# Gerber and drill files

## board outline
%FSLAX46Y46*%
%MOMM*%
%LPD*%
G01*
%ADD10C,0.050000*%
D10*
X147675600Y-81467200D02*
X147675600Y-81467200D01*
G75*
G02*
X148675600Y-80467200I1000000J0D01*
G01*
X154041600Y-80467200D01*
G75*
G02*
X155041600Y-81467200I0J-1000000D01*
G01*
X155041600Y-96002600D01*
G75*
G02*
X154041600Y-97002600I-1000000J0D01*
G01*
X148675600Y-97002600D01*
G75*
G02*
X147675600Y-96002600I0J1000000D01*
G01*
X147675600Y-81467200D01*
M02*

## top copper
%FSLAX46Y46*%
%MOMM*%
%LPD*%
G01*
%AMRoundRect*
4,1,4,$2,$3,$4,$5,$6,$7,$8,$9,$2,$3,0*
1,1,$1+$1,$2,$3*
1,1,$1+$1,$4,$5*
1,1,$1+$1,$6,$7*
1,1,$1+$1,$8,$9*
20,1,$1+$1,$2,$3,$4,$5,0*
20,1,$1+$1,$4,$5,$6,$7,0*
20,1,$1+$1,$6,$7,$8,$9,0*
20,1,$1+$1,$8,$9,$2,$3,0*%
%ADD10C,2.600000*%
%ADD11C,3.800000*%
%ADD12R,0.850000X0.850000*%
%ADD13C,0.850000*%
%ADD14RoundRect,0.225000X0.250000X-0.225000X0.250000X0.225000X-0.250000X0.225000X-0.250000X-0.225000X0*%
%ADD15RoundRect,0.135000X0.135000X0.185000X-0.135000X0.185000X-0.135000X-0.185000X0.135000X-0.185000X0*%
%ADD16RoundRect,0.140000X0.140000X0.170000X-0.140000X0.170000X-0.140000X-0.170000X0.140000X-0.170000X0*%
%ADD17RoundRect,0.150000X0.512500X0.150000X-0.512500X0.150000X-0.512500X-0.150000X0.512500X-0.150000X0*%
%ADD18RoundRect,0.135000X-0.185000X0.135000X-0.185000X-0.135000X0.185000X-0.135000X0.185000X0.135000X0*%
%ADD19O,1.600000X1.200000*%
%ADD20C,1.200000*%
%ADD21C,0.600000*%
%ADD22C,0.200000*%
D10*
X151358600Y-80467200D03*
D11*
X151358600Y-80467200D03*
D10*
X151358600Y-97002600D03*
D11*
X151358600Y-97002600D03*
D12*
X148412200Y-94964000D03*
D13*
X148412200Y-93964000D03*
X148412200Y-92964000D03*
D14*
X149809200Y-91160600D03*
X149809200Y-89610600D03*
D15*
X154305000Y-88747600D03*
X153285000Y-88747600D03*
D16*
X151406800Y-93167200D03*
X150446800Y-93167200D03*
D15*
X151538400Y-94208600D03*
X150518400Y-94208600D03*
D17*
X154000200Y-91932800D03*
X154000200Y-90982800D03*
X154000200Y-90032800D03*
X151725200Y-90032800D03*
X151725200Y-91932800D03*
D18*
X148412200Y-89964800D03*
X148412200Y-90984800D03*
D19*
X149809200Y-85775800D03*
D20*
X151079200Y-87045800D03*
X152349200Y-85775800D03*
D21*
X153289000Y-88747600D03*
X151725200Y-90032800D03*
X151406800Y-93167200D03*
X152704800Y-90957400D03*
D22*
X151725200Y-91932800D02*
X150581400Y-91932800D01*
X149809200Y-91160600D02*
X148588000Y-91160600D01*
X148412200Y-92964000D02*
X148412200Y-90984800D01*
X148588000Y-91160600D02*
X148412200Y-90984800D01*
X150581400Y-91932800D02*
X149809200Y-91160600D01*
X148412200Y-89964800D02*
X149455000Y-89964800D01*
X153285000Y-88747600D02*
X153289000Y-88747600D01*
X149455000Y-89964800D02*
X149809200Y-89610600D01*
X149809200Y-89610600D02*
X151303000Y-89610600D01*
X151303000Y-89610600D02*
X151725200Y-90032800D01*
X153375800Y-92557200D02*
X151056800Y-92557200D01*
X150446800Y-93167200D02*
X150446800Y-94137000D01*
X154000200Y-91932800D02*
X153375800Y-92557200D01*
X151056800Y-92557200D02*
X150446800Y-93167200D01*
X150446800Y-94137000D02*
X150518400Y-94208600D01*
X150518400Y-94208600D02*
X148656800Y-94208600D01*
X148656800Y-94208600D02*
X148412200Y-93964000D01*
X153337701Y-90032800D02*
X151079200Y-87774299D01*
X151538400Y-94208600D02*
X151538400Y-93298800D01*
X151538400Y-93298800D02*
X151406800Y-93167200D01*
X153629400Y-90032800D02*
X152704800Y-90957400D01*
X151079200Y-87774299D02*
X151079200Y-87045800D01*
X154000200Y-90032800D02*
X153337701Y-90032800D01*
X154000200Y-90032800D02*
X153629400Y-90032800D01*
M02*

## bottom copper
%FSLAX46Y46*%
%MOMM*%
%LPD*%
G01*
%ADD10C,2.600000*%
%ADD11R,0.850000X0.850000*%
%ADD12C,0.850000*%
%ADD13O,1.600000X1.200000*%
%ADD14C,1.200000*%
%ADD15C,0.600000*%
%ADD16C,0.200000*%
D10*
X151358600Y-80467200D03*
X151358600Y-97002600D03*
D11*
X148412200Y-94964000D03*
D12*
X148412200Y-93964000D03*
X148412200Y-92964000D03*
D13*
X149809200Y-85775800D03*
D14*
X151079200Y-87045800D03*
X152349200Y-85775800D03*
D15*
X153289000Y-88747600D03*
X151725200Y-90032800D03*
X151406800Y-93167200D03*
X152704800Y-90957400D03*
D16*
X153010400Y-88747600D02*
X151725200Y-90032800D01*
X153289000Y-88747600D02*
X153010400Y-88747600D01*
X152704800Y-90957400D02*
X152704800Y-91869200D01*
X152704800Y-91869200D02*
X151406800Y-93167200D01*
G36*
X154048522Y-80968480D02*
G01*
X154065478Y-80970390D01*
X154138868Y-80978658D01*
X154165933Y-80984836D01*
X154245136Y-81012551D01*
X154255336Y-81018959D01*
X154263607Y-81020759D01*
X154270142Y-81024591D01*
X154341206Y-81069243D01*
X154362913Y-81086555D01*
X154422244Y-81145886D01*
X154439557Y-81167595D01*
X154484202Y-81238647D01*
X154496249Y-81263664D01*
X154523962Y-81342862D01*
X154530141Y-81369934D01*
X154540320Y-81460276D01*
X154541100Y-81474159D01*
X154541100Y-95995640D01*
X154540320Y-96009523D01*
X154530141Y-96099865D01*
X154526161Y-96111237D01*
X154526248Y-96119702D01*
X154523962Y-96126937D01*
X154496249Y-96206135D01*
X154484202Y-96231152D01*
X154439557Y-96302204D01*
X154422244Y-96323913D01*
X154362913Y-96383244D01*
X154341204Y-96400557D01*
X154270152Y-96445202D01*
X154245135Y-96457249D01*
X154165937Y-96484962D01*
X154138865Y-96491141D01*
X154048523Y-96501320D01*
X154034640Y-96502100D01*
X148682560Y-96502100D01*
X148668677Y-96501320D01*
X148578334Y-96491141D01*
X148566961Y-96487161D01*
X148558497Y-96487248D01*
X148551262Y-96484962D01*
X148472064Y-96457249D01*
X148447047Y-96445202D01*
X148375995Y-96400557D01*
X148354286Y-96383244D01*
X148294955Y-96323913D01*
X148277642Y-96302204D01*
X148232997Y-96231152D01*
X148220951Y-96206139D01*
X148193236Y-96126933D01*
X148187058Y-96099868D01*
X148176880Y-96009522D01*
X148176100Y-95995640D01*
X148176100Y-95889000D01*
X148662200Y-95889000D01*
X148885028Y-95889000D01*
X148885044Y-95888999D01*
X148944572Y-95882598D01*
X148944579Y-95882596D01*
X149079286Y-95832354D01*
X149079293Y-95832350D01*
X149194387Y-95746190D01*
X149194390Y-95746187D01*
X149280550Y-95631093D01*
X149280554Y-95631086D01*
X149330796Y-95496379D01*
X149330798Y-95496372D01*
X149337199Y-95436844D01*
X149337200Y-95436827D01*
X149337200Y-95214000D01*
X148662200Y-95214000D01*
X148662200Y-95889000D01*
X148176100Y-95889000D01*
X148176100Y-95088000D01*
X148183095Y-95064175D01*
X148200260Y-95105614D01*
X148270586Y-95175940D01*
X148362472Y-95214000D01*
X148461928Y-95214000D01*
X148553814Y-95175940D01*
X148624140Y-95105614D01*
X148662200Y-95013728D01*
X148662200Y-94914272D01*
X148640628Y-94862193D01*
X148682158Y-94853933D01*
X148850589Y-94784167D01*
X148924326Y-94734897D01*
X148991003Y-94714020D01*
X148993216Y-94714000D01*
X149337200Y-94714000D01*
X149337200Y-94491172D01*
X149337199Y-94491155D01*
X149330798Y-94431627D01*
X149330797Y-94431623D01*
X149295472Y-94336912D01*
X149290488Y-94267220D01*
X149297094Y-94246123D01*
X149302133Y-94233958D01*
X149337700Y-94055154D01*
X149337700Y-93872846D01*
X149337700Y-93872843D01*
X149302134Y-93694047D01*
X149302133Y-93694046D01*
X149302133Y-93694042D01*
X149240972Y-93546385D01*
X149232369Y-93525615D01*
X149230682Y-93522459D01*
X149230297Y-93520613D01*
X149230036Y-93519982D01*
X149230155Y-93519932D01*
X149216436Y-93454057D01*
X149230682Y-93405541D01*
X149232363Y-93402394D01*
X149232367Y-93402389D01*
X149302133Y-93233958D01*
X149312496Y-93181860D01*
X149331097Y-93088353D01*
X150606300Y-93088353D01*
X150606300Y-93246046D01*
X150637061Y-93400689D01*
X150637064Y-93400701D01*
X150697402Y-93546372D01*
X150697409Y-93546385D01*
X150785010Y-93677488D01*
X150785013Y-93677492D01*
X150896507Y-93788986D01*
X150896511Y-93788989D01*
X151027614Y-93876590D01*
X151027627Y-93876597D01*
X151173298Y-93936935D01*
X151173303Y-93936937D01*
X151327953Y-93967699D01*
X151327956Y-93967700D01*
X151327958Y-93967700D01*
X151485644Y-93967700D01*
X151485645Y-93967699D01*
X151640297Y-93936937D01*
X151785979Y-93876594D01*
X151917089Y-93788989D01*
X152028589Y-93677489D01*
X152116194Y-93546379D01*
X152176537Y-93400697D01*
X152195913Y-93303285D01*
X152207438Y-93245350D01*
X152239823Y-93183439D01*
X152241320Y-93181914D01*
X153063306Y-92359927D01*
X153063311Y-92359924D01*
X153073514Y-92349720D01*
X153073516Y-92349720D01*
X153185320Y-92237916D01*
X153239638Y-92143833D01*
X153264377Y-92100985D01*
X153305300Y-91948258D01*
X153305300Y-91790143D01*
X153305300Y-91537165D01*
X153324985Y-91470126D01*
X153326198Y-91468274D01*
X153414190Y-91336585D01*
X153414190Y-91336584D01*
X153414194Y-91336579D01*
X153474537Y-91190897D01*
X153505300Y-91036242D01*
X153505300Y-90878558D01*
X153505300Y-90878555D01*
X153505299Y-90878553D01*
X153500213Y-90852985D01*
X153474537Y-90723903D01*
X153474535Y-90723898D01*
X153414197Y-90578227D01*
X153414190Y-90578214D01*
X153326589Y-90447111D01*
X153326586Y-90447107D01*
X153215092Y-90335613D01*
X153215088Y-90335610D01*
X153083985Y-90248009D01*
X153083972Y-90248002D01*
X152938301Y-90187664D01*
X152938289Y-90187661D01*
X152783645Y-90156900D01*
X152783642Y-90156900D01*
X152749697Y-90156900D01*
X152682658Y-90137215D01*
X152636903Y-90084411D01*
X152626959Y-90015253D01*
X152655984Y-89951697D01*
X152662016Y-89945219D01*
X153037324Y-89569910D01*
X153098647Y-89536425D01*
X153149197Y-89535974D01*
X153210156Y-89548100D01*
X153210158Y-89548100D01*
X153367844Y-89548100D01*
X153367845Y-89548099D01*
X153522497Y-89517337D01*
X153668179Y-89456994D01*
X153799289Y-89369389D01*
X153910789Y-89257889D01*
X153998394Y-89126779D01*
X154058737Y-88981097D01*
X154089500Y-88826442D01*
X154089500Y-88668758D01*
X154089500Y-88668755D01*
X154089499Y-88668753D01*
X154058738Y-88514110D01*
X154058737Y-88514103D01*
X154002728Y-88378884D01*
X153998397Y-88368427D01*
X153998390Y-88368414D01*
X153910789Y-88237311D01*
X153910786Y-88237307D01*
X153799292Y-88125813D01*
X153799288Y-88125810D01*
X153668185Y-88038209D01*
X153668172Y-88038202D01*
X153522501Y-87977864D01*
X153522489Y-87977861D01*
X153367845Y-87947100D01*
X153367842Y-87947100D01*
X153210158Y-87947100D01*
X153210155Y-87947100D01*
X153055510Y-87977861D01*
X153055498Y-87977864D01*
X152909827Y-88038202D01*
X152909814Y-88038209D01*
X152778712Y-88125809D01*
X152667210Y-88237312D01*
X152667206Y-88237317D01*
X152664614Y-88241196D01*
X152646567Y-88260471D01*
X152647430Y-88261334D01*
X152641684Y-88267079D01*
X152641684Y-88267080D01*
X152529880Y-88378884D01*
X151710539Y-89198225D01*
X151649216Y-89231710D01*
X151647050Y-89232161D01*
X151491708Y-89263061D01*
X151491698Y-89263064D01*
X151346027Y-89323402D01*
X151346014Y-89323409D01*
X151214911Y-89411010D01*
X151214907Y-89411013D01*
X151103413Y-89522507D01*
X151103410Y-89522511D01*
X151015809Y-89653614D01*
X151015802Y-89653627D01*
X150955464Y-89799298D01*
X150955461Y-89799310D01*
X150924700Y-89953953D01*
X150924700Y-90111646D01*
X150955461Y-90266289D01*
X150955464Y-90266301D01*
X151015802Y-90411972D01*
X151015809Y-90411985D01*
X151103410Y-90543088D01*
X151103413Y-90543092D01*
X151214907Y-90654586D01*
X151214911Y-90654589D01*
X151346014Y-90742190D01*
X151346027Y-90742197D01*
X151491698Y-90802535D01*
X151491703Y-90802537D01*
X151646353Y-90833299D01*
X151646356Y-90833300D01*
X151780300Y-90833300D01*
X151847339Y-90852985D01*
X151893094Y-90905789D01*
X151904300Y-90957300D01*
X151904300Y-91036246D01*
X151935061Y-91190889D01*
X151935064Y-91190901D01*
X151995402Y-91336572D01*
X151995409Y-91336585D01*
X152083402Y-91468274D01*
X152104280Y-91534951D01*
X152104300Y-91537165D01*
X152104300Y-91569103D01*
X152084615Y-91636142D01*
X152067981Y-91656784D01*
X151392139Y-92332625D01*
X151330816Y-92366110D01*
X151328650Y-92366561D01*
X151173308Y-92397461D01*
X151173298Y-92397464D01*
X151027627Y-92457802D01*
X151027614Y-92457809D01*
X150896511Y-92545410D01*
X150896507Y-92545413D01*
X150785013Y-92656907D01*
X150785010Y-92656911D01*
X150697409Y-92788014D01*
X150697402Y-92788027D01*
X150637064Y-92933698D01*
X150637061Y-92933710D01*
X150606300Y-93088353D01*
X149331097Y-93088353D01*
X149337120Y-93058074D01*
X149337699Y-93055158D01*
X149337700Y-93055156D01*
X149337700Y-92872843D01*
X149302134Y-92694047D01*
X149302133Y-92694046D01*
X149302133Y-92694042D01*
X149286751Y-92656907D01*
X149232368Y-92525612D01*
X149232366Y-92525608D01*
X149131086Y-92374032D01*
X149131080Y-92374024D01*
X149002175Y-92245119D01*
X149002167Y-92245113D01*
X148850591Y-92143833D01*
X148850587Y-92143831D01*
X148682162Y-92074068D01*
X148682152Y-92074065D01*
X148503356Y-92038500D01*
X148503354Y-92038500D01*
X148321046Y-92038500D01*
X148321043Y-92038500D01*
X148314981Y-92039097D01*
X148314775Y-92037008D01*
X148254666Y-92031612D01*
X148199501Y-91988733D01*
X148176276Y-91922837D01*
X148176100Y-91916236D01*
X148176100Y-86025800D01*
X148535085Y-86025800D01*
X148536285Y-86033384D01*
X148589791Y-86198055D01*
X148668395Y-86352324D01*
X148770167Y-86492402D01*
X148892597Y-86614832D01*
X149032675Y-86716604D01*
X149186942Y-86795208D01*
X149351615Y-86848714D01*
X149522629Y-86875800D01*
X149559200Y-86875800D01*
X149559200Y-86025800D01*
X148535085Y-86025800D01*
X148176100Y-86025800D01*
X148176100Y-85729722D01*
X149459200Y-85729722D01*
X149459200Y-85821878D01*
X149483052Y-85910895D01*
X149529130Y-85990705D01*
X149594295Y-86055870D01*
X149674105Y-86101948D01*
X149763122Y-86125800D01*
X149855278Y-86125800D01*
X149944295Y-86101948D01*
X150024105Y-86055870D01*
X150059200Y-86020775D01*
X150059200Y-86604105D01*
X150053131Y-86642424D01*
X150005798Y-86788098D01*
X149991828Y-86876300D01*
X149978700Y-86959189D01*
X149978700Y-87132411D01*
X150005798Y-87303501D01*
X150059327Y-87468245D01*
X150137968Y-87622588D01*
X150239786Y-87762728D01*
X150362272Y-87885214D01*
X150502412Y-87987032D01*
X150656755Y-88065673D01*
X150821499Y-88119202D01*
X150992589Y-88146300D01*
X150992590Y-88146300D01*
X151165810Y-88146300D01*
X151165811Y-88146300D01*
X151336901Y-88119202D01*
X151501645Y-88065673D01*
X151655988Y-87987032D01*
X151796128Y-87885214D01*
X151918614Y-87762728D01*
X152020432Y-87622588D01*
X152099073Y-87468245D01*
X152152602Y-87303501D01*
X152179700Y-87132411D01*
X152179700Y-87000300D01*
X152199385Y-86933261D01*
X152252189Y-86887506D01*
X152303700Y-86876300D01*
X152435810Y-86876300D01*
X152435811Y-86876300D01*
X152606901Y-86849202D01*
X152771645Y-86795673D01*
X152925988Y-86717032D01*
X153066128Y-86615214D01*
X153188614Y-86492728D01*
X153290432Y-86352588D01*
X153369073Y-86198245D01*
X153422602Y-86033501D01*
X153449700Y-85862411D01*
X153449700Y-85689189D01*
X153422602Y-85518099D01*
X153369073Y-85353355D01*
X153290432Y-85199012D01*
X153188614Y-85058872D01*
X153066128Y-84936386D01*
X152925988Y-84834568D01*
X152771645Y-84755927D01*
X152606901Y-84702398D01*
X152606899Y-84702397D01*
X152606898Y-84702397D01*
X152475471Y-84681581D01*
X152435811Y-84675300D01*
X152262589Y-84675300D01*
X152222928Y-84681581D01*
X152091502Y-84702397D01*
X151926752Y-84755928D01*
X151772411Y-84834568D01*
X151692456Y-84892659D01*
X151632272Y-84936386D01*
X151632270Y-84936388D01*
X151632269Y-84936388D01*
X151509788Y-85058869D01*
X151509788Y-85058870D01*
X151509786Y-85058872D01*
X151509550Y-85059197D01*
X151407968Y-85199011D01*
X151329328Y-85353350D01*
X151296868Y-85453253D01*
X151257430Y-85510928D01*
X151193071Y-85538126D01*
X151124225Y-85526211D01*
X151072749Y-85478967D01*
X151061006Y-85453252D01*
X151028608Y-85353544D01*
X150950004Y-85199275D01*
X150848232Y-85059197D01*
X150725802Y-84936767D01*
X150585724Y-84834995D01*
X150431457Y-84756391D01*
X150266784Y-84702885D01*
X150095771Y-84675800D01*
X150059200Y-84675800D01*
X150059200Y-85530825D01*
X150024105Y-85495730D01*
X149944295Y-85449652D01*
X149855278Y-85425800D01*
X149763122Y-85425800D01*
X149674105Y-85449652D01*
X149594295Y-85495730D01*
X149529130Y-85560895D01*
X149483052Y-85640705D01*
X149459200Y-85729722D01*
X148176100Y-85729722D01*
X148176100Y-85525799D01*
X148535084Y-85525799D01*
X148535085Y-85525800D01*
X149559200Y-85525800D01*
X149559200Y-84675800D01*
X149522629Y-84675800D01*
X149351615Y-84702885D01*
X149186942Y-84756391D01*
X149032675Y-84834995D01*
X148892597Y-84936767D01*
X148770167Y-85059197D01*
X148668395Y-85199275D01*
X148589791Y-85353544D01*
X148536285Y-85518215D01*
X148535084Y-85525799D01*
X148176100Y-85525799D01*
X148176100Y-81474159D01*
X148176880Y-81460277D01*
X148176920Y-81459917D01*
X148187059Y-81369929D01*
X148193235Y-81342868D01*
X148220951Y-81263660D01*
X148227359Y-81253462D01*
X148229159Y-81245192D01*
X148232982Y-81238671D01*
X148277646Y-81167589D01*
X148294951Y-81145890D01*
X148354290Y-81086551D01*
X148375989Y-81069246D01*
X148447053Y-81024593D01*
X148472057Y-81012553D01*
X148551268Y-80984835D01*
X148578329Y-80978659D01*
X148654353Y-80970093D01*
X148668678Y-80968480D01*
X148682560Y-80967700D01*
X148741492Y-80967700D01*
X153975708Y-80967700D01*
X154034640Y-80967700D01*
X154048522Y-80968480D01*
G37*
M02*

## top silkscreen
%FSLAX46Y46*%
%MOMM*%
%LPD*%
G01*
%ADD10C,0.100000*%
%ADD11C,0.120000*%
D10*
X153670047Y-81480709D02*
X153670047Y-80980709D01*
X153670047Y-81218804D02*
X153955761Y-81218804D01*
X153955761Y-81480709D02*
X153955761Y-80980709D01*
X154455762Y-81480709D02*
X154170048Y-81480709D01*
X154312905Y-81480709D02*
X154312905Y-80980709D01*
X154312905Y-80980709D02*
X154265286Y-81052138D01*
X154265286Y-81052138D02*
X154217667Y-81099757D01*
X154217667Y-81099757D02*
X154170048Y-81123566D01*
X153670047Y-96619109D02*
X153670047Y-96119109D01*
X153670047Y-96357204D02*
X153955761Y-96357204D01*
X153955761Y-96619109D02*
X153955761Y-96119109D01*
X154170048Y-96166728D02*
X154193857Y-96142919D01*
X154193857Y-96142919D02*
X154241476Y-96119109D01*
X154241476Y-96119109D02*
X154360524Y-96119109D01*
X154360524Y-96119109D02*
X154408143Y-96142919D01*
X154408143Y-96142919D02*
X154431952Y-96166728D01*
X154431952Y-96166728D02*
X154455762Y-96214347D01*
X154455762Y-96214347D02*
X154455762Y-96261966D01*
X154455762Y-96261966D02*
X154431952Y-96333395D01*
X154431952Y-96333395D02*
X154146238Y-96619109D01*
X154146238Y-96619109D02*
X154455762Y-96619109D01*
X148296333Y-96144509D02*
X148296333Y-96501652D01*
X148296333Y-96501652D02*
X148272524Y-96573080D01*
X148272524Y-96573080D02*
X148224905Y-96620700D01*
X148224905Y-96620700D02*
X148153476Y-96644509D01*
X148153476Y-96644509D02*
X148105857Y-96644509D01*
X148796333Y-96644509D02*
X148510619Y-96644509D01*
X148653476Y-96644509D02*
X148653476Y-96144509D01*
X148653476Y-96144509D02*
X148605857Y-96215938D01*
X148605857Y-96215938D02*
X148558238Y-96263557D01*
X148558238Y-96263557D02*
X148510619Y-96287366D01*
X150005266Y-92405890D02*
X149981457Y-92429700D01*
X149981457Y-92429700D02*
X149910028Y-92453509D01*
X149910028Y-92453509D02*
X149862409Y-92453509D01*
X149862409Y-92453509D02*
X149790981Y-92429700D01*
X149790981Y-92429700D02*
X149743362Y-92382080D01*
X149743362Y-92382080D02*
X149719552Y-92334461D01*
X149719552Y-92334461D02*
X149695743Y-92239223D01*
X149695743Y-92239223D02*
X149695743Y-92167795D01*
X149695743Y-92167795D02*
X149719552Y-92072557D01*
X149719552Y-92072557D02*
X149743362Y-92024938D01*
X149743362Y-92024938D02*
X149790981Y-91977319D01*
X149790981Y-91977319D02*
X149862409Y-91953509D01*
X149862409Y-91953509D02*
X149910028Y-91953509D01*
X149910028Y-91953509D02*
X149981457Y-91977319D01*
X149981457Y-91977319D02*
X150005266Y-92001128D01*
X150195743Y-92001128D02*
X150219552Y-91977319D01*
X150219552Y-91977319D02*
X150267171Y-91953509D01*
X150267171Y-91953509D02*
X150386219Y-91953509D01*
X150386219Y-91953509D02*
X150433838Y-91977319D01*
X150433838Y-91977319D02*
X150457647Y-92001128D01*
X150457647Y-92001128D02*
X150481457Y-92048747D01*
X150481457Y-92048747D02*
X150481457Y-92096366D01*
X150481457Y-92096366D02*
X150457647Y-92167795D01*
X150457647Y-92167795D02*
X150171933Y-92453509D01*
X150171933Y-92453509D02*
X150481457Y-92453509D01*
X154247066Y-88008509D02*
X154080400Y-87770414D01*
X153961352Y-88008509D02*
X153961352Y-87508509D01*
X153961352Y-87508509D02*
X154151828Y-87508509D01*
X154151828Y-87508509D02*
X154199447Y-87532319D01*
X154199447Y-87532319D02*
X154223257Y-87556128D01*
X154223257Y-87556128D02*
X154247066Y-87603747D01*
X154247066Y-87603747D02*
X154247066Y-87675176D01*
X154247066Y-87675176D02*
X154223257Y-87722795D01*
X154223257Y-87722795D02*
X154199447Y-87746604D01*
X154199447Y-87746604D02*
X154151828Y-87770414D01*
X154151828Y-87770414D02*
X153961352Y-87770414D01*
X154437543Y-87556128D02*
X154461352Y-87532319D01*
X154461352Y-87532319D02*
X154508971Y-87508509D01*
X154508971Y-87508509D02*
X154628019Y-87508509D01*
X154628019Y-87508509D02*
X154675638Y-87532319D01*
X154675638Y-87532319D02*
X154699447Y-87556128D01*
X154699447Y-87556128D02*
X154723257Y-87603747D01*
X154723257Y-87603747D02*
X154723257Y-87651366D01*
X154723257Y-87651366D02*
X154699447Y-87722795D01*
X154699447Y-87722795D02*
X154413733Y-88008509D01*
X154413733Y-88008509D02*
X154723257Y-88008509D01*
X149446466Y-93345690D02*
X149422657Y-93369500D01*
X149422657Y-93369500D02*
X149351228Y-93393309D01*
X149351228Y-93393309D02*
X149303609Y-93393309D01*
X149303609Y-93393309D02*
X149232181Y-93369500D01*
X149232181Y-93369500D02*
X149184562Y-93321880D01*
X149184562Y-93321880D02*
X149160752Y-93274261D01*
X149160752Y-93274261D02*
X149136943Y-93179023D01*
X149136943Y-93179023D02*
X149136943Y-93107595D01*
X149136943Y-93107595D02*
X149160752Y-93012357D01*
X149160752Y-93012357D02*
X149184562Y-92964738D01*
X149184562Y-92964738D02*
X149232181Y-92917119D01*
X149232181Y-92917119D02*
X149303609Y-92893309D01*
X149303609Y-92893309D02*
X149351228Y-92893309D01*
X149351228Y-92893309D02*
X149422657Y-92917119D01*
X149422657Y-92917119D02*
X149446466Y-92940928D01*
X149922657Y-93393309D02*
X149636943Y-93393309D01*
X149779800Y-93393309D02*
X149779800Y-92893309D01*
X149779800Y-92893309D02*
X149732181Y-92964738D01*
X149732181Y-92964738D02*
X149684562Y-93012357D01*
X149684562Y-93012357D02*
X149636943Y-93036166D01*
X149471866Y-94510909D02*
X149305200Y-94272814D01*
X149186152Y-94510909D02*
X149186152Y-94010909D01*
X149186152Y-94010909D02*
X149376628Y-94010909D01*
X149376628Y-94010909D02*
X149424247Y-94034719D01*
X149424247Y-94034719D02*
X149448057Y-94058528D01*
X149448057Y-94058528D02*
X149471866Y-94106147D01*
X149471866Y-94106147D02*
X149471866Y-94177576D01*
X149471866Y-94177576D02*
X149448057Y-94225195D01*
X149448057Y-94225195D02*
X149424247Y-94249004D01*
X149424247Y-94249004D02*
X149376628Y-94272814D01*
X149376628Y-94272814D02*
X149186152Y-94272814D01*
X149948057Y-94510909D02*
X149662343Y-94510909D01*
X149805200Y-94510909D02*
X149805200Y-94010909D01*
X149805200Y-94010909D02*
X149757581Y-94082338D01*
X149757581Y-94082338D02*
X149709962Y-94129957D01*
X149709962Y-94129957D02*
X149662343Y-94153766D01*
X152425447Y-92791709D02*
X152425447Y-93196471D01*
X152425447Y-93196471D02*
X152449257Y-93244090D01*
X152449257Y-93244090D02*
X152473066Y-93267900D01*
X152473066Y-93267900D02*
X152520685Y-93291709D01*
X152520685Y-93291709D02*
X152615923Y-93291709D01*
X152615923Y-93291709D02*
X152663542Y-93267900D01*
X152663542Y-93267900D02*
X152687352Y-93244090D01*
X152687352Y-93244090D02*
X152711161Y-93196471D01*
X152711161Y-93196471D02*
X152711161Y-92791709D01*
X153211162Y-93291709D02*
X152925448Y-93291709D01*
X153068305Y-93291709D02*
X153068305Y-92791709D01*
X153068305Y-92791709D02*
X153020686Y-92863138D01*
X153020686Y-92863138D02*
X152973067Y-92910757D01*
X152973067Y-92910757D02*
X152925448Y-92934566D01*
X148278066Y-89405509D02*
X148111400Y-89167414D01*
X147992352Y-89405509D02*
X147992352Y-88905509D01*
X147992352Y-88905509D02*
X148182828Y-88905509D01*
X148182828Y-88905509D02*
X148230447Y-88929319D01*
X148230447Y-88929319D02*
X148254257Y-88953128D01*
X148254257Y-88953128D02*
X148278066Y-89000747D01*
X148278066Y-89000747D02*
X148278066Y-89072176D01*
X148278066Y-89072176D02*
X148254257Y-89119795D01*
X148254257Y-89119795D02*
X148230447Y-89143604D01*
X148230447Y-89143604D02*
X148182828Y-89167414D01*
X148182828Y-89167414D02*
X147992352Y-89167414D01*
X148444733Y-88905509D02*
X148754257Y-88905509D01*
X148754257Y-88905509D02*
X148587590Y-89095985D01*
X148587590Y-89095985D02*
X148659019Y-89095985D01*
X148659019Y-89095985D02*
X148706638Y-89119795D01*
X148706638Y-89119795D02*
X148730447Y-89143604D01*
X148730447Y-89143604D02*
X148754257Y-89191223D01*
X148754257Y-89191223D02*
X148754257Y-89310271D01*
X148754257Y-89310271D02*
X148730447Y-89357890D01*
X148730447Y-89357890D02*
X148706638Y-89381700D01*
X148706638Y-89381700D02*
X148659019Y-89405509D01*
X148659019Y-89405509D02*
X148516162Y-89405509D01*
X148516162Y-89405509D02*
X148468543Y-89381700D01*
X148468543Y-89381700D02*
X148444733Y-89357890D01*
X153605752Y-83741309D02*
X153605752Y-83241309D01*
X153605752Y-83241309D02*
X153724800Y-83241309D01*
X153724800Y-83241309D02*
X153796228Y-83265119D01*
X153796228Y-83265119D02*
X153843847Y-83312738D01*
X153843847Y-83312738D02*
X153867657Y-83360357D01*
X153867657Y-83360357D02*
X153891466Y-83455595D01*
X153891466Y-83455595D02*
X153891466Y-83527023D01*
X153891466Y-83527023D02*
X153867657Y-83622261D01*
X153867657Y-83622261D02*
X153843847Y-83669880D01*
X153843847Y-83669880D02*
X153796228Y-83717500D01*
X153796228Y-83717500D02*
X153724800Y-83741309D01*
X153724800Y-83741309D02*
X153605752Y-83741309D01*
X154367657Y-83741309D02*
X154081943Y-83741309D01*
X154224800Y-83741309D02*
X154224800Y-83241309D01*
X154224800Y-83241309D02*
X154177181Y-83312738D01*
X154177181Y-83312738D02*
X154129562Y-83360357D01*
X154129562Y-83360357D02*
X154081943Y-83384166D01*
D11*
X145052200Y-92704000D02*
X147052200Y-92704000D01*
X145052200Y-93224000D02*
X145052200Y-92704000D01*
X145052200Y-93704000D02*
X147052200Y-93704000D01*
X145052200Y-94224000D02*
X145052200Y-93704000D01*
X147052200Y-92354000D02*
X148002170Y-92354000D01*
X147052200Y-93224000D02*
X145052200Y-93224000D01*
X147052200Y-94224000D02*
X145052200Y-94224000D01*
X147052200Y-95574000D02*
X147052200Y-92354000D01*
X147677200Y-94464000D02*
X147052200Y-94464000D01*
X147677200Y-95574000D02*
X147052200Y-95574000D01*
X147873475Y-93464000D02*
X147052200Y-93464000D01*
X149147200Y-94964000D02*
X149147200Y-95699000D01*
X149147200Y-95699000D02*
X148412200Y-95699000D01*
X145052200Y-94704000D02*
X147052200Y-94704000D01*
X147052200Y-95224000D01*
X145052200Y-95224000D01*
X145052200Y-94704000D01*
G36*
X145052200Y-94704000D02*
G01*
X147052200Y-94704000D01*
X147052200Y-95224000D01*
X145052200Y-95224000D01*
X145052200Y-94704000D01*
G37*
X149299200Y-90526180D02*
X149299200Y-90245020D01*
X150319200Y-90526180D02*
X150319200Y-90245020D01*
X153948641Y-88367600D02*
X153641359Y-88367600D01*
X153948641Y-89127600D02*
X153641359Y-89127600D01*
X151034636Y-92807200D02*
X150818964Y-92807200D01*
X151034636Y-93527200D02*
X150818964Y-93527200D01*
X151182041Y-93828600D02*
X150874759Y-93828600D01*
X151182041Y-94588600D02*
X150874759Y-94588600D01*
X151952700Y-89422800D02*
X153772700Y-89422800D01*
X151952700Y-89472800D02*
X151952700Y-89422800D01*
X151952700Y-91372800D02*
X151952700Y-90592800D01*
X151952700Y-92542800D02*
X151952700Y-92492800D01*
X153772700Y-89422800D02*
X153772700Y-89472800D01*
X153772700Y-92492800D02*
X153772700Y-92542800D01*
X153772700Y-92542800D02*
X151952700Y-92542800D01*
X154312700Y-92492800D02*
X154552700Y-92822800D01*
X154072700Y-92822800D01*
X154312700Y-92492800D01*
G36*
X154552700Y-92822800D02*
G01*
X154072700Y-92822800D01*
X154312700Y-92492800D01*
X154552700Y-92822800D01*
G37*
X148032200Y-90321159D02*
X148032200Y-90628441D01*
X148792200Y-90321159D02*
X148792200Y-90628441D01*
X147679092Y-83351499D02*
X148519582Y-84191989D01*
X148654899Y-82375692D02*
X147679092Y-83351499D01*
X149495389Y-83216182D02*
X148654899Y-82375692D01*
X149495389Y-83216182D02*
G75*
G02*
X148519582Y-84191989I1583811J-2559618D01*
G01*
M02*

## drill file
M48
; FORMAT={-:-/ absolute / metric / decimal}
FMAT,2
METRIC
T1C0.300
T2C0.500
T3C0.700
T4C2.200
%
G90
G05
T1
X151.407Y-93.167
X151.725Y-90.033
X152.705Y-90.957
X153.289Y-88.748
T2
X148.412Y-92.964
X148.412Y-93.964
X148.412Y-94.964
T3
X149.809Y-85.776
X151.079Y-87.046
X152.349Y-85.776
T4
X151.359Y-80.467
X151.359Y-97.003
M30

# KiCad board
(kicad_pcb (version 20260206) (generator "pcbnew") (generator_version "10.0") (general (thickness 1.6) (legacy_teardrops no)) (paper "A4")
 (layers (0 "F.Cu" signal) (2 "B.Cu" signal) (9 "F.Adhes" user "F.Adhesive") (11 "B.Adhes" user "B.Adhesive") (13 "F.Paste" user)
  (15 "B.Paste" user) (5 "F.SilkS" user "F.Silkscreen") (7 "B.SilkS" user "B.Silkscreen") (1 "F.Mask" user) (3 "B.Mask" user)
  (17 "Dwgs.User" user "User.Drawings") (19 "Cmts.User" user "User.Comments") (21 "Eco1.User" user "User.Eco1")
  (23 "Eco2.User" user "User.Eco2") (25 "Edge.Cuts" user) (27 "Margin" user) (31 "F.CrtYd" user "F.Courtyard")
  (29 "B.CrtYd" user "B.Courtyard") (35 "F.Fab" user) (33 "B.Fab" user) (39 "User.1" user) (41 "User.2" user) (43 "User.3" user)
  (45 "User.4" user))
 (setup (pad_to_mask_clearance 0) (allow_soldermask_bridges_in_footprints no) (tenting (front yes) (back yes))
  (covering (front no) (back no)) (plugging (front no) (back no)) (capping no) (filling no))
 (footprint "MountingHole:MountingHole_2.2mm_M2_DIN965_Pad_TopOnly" (layer "F.Cu") (at 151.3586 80.4672)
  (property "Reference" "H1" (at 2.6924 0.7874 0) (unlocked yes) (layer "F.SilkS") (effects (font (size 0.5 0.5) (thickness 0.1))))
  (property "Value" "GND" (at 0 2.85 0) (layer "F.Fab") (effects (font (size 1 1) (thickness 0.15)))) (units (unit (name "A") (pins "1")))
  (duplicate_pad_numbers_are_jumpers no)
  (pad "1" thru_hole circle (at 0 0) (size 2.6 2.6) (drill 2.2) (layers "*.Cu" "*.Mask") (remove_unused_layers no) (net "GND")
   (zone_connect 2))
  (pad "1" connect circle (at 0 0) (size 3.8 3.8) (layers "F.Cu" "F.Mask") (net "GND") (zone_connect 2)))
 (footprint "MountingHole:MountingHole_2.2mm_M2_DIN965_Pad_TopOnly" (layer "F.Cu") (at 151.3586 97.0026)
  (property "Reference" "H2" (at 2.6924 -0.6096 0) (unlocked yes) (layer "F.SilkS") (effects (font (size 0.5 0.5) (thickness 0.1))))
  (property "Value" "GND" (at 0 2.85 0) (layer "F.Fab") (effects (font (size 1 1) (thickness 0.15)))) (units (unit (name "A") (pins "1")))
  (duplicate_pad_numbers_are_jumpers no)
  (pad "1" thru_hole circle (at 0 0) (size 2.6 2.6) (drill 2.2) (layers "*.Cu" "*.Mask") (remove_unused_layers no) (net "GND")
   (zone_connect 2))
  (pad "1" connect circle (at 0 0) (size 3.8 3.8) (layers "F.Cu" "F.Mask") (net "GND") (zone_connect 2)))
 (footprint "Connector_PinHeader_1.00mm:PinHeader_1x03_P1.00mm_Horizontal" (layer "F.Cu") (at 148.4122 94.964 180)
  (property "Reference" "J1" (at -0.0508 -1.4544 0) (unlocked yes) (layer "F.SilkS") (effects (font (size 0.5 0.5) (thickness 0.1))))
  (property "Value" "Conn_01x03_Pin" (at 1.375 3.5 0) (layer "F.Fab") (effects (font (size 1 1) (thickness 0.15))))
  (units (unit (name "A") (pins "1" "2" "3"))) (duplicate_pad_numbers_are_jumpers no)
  (fp_line (start 3.36 2.26) (end 1.36 2.26) (stroke (width 0.12) (type solid)) (layer "F.SilkS"))
  (fp_line (start 3.36 1.74) (end 3.36 2.26) (stroke (width 0.12) (type solid)) (layer "F.SilkS"))
  (fp_line (start 3.36 1.26) (end 1.36 1.26) (stroke (width 0.12) (type solid)) (layer "F.SilkS"))
  (fp_line (start 3.36 0.74) (end 3.36 1.26) (stroke (width 0.12) (type solid)) (layer "F.SilkS"))
  (fp_line (start 1.36 2.61) (end 0.41003 2.61) (stroke (width 0.12) (type solid)) (layer "F.SilkS"))
  (fp_line (start 1.36 1.74) (end 3.36 1.74) (stroke (width 0.12) (type solid)) (layer "F.SilkS"))
  (fp_line (start 1.36 0.74) (end 3.36 0.74) (stroke (width 0.12) (type solid)) (layer "F.SilkS"))
  (fp_line (start 1.36 -0.61) (end 1.36 2.61) (stroke (width 0.12) (type solid)) (layer "F.SilkS"))
  (fp_line (start 0.735 0.5) (end 1.36 0.5) (stroke (width 0.12) (type solid)) (layer "F.SilkS"))
  (fp_line (start 0.735 -0.61) (end 1.36 -0.61) (stroke (width 0.12) (type solid)) (layer "F.SilkS"))
  (fp_line (start 0.538725 1.5) (end 1.36 1.5) (stroke (width 0.12) (type solid)) (layer "F.SilkS"))
  (fp_line (start -0.735 0) (end -0.735 -0.735) (stroke (width 0.12) (type solid)) (layer "F.SilkS"))
  (fp_line (start -0.735 -0.735) (end 0 -0.735) (stroke (width 0.12) (type solid)) (layer "F.SilkS"))
  (fp_rect (start 1.36 -0.26) (end 3.36 0.26) (stroke (width 0.12) (type solid)) (fill yes) (layer "F.SilkS"))
  (pad "1" thru_hole rect (at 0 0 180) (size 0.85 0.85) (drill 0.5) (layers "*.Cu" "*.Mask") (remove_unused_layers no) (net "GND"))
  (pad "2" thru_hole circle (at 0 1 180) (size 0.85 0.85) (drill 0.5) (layers "*.Cu" "*.Mask") (remove_unused_layers no)
   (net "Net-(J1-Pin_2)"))
  (pad "3" thru_hole circle (at 0 2 180) (size 0.85 0.85) (drill 0.5) (layers "*.Cu" "*.Mask") (remove_unused_layers no) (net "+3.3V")))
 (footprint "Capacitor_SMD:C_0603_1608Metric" (layer "F.Cu") (at 149.8092 90.3856 90)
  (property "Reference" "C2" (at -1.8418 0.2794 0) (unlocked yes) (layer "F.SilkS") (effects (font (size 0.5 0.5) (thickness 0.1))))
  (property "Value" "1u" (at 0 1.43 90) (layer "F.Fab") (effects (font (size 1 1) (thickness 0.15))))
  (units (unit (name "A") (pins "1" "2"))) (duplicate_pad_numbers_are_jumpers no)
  (fp_line (start -0.14058 -0.51) (end 0.14058 -0.51) (stroke (width 0.12) (type solid)) (layer "F.SilkS"))
  (fp_line (start -0.14058 0.51) (end 0.14058 0.51) (stroke (width 0.12) (type solid)) (layer "F.SilkS"))
  (pad "1" smd roundrect (at -0.775 0 90) (size 0.9 0.95) (layers "F.Cu" "F.Mask" "F.Paste") (roundrect_rratio 0.25) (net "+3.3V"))
  (pad "2" smd roundrect (at 0.775 0 90) (size 0.9 0.95) (layers "F.Cu" "F.Mask" "F.Paste") (roundrect_rratio 0.25) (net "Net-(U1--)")))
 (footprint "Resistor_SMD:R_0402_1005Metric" (layer "F.Cu") (at 153.795 88.7476 180)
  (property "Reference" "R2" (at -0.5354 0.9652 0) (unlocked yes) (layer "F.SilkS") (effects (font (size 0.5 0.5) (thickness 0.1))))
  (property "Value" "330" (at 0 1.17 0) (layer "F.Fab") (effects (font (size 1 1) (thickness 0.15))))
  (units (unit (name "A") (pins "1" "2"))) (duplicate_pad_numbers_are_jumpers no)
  (fp_line (start -0.153641 0.38) (end 0.153641 0.38) (stroke (width 0.12) (type solid)) (layer "F.SilkS"))
  (fp_line (start -0.153641 -0.38) (end 0.153641 -0.38) (stroke (width 0.12) (type solid)) (layer "F.SilkS"))
  (pad "1" smd roundrect (at -0.51 0 180) (size 0.54 0.64) (layers "F.Cu" "F.Mask" "F.Paste") (roundrect_rratio 0.25) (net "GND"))
  (pad "2" smd roundrect (at 0.51 0 180) (size 0.54 0.64) (layers "F.Cu" "F.Mask" "F.Paste") (roundrect_rratio 0.25) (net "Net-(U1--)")))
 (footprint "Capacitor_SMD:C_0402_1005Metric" (layer "F.Cu") (at 150.9268 93.1672 180)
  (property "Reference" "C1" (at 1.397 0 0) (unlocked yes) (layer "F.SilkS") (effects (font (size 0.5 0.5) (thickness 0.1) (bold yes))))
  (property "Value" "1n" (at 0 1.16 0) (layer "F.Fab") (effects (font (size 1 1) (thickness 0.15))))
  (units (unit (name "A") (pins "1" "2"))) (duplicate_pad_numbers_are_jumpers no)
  (fp_line (start -0.107836 0.36) (end 0.107836 0.36) (stroke (width 0.12) (type solid)) (layer "F.SilkS"))
  (fp_line (start -0.107836 -0.36) (end 0.107836 -0.36) (stroke (width 0.12) (type solid)) (layer "F.SilkS"))
  (pad "1" smd roundrect (at -0.48 0 180) (size 0.56 0.62) (layers "F.Cu" "F.Mask" "F.Paste") (roundrect_rratio 0.25) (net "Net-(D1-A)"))
  (pad "2" smd roundrect (at 0.48 0 180) (size 0.56 0.62) (layers "F.Cu" "F.Mask" "F.Paste") (roundrect_rratio 0.25) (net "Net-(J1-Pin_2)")))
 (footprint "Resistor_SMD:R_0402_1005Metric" (layer "F.Cu") (at 151.0284 94.2086 180)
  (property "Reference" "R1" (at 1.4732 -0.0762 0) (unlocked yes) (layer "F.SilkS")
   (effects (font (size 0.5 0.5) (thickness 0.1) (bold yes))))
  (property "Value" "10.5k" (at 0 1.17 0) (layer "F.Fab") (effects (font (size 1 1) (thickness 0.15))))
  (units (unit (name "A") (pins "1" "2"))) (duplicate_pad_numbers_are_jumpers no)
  (fp_line (start -0.153641 0.38) (end 0.153641 0.38) (stroke (width 0.12) (type solid)) (layer "F.SilkS"))
  (fp_line (start -0.153641 -0.38) (end 0.153641 -0.38) (stroke (width 0.12) (type solid)) (layer "F.SilkS"))
  (pad "1" smd roundrect (at -0.51 0 180) (size 0.54 0.64) (layers "F.Cu" "F.Mask" "F.Paste") (roundrect_rratio 0.25) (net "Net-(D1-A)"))
  (pad "2" smd roundrect (at 0.51 0 180) (size 0.54 0.64) (layers "F.Cu" "F.Mask" "F.Paste") (roundrect_rratio 0.25) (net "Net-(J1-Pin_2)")))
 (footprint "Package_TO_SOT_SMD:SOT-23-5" (layer "F.Cu") (at 152.8627 90.9828 180)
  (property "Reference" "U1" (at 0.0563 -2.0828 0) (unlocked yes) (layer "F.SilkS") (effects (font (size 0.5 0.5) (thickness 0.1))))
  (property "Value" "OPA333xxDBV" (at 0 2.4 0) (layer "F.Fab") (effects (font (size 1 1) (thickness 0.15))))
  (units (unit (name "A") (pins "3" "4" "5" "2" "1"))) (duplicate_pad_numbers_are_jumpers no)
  (fp_line (start 0.91 1.56) (end -0.91 1.56) (stroke (width 0.12) (type solid)) (layer "F.SilkS"))
  (fp_line (start 0.91 1.51) (end 0.91 1.56) (stroke (width 0.12) (type solid)) (layer "F.SilkS"))
  (fp_line (start 0.91 -0.39) (end 0.91 0.39) (stroke (width 0.12) (type solid)) (layer "F.SilkS"))
  (fp_line (start 0.91 -1.56) (end 0.91 -1.51) (stroke (width 0.12) (type solid)) (layer "F.SilkS"))
  (fp_line (start -0.91 1.56) (end -0.91 1.51) (stroke (width 0.12) (type solid)) (layer "F.SilkS"))
  (fp_line (start -0.91 -1.51) (end -0.91 -1.56) (stroke (width 0.12) (type solid)) (layer "F.SilkS"))
  (fp_line (start -0.91 -1.56) (end 0.91 -1.56) (stroke (width 0.12) (type solid)) (layer "F.SilkS"))
  (fp_poly (pts (xy -1.45 -1.51) (xy -1.69 -1.84) (xy -1.21 -1.84)) (stroke (width 0.12) (type solid)) (fill yes) (layer "F.SilkS"))
  (pad "1" smd roundrect (at -1.1375 -0.95 180) (size 1.325 0.6) (layers "F.Cu" "F.Mask" "F.Paste") (roundrect_rratio 0.25)
   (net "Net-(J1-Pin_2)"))
  (pad "2" smd roundrect (at -1.1375 0 180) (size 1.325 0.6) (layers "F.Cu" "F.Mask" "F.Paste") (roundrect_rratio 0.25) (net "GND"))
  (pad "3" smd roundrect (at -1.1375 0.95 180) (size 1.325 0.6) (layers "F.Cu" "F.Mask" "F.Paste") (roundrect_rratio 0.25)
   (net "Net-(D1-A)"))
  (pad "4" smd roundrect (at 1.1375 0.95 180) (size 1.325 0.6) (layers "F.Cu" "F.Mask" "F.Paste") (roundrect_rratio 0.25) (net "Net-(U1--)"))
  (pad "5" smd roundrect (at 1.1375 -0.95 180) (size 1.325 0.6) (layers "F.Cu" "F.Mask" "F.Paste") (roundrect_rratio 0.25) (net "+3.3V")))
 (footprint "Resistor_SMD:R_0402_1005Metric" (layer "F.Cu") (at 148.4122 90.4748 -90)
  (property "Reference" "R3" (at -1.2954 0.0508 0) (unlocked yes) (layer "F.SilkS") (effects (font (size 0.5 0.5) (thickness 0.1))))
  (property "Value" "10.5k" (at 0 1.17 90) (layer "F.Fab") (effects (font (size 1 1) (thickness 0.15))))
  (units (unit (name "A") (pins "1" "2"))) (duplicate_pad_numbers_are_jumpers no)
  (fp_line (start -0.153641 0.38) (end 0.153641 0.38) (stroke (width 0.12) (type solid)) (layer "F.SilkS"))
  (fp_line (start -0.153641 -0.38) (end 0.153641 -0.38) (stroke (width 0.12) (type solid)) (layer "F.SilkS"))
  (pad "1" smd roundrect (at -0.51 0 270) (size 0.54 0.64) (layers "F.Cu" "F.Mask" "F.Paste") (roundrect_rratio 0.25) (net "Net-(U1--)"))
  (pad "2" smd roundrect (at 0.51 0 270) (size 0.54 0.64) (layers "F.Cu" "F.Mask" "F.Paste") (roundrect_rratio 0.25) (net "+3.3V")))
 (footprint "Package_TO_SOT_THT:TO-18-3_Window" (layer "F.Cu") (at 149.8092 85.7758)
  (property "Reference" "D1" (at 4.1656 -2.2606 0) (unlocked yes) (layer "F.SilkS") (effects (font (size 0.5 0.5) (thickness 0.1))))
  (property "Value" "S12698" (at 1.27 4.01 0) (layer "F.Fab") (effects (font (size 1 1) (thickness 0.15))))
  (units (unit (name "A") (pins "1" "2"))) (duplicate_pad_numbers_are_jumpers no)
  (fp_line (start -2.130108 -2.424301) (end -1.289618 -1.583811) (stroke (width 0.12) (type solid)) (layer "F.SilkS"))
  (fp_line (start -1.154301 -3.400108) (end -2.130108 -2.424301) (stroke (width 0.12) (type solid)) (layer "F.SilkS"))
  (fp_line (start -0.313811 -2.559618) (end -1.154301 -3.400108) (stroke (width 0.12) (type solid)) (layer "F.SilkS"))
  (fp_arc (start -0.313811 -2.559618) (mid 3.398391 2.128391) (end -1.289618 -1.583811) (stroke (width 0.12) (type solid)) (layer "F.SilkS"))
  (pad "1" thru_hole oval (at 0 0) (size 1.6 1.2) (drill 0.7) (layers "*.Cu" "*.Mask") (remove_unused_layers no) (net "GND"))
  (pad "2" thru_hole circle (at 1.27 1.27) (size 1.2 1.2) (drill 0.7) (layers "*.Cu" "*.Mask") (remove_unused_layers no) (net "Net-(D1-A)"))
  (pad "3" thru_hole circle (at 2.54 0) (size 1.2 1.2) (drill 0.7) (layers "*.Cu" "*.Mask") (remove_unused_layers no)))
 (gr_rect (start 147.6756 80.4672) (end 155.0416 97.0026) (radius 1) (stroke (width 0.05) (type solid)) (fill no) (layer "Edge.Cuts"))
 (segment (start 151.7252 91.9328) (end 150.5814 91.9328) (width 0.2) (layer "F.Cu") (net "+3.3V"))
 (segment (start 149.8092 91.1606) (end 148.588 91.1606) (width 0.2) (layer "F.Cu") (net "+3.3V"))
 (segment (start 148.4122 92.964) (end 148.4122 90.9848) (width 0.2) (layer "F.Cu") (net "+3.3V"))
 (segment (start 148.588 91.1606) (end 148.4122 90.9848) (width 0.2) (layer "F.Cu") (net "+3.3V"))
 (segment (start 150.5814 91.9328) (end 149.8092 91.1606) (width 0.2) (layer "F.Cu") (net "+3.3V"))
 (segment (start 148.4122 89.9648) (end 149.455 89.9648) (width 0.2) (layer "F.Cu") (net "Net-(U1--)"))
 (segment (start 153.285 88.7476) (end 153.289 88.7476) (width 0.2) (layer "F.Cu") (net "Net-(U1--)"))
 (segment (start 149.455 89.9648) (end 149.8092 89.6106) (width 0.2) (layer "F.Cu") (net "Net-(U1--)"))
 (segment (start 149.8092 89.6106) (end 151.303 89.6106) (width 0.2) (layer "F.Cu") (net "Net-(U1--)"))
 (segment (start 151.303 89.6106) (end 151.7252 90.0328) (width 0.2) (layer "F.Cu") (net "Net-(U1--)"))
 (via (at 153.289 88.7476) (size 0.6) (drill 0.3) (layers "F.Cu" "B.Cu") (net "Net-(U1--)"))
 (via (at 151.7252 90.0328) (size 0.6) (drill 0.3) (layers "F.Cu" "B.Cu") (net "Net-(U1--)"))
 (segment (start 153.0104 88.7476) (end 151.7252 90.0328) (width 0.2) (layer "B.Cu") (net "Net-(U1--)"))
 (segment (start 153.289 88.7476) (end 153.0104 88.7476) (width 0.2) (layer "B.Cu") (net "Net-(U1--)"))
 (segment (start 153.3758 92.5572) (end 151.0568 92.5572) (width 0.2) (layer "F.Cu") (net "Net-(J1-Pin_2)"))
 (segment (start 150.4468 93.1672) (end 150.4468 94.137) (width 0.2) (layer "F.Cu") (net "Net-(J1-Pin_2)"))
 (segment (start 154.0002 91.9328) (end 153.3758 92.5572) (width 0.2) (layer "F.Cu") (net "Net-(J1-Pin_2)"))
 (segment (start 151.0568 92.5572) (end 150.4468 93.1672) (width 0.2) (layer "F.Cu") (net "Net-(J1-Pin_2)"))
 (segment (start 150.4468 94.137) (end 150.5184 94.2086) (width 0.2) (layer "F.Cu") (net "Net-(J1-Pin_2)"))
 (segment (start 150.5184 94.2086) (end 148.6568 94.2086) (width 0.2) (layer "F.Cu") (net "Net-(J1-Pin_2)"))
 (segment (start 148.6568 94.2086) (end 148.4122 93.964) (width 0.2) (layer "F.Cu") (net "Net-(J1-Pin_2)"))
 (segment (start 153.337701 90.0328) (end 151.0792 87.774299) (width 0.2) (layer "F.Cu") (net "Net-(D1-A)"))
 (segment (start 151.5384 94.2086) (end 151.5384 93.2988) (width 0.2) (layer "F.Cu") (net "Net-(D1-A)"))
 (segment (start 151.5384 93.2988) (end 151.4068 93.1672) (width 0.2) (layer "F.Cu") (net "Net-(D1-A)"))
 (segment (start 153.6294 90.0328) (end 152.7048 90.9574) (width 0.2) (layer "F.Cu") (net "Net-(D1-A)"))
 (segment (start 151.0792 87.774299) (end 151.0792 87.0458) (width 0.2) (layer "F.Cu") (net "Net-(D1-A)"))
 (segment (start 154.0002 90.0328) (end 153.337701 90.0328) (width 0.2) (layer "F.Cu") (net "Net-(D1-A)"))
 (segment (start 154.0002 90.0328) (end 153.6294 90.0328) (width 0.2) (layer "F.Cu") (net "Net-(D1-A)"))
 (via (at 151.4068 93.1672) (size 0.6) (drill 0.3) (layers "F.Cu" "B.Cu") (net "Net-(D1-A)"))
 (via (at 152.7048 90.9574) (size 0.6) (drill 0.3) (layers "F.Cu" "B.Cu") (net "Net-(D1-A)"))
 (segment (start 152.7048 90.9574) (end 152.7048 91.8692) (width 0.2) (layer "B.Cu") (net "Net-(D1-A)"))
 (segment (start 152.7048 91.8692) (end 151.4068 93.1672) (width 0.2) (layer "B.Cu") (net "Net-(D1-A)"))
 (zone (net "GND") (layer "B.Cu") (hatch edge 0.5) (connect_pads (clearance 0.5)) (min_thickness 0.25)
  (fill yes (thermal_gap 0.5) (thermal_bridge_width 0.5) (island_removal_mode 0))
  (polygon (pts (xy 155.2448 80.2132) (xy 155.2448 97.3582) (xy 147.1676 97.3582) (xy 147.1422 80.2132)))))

